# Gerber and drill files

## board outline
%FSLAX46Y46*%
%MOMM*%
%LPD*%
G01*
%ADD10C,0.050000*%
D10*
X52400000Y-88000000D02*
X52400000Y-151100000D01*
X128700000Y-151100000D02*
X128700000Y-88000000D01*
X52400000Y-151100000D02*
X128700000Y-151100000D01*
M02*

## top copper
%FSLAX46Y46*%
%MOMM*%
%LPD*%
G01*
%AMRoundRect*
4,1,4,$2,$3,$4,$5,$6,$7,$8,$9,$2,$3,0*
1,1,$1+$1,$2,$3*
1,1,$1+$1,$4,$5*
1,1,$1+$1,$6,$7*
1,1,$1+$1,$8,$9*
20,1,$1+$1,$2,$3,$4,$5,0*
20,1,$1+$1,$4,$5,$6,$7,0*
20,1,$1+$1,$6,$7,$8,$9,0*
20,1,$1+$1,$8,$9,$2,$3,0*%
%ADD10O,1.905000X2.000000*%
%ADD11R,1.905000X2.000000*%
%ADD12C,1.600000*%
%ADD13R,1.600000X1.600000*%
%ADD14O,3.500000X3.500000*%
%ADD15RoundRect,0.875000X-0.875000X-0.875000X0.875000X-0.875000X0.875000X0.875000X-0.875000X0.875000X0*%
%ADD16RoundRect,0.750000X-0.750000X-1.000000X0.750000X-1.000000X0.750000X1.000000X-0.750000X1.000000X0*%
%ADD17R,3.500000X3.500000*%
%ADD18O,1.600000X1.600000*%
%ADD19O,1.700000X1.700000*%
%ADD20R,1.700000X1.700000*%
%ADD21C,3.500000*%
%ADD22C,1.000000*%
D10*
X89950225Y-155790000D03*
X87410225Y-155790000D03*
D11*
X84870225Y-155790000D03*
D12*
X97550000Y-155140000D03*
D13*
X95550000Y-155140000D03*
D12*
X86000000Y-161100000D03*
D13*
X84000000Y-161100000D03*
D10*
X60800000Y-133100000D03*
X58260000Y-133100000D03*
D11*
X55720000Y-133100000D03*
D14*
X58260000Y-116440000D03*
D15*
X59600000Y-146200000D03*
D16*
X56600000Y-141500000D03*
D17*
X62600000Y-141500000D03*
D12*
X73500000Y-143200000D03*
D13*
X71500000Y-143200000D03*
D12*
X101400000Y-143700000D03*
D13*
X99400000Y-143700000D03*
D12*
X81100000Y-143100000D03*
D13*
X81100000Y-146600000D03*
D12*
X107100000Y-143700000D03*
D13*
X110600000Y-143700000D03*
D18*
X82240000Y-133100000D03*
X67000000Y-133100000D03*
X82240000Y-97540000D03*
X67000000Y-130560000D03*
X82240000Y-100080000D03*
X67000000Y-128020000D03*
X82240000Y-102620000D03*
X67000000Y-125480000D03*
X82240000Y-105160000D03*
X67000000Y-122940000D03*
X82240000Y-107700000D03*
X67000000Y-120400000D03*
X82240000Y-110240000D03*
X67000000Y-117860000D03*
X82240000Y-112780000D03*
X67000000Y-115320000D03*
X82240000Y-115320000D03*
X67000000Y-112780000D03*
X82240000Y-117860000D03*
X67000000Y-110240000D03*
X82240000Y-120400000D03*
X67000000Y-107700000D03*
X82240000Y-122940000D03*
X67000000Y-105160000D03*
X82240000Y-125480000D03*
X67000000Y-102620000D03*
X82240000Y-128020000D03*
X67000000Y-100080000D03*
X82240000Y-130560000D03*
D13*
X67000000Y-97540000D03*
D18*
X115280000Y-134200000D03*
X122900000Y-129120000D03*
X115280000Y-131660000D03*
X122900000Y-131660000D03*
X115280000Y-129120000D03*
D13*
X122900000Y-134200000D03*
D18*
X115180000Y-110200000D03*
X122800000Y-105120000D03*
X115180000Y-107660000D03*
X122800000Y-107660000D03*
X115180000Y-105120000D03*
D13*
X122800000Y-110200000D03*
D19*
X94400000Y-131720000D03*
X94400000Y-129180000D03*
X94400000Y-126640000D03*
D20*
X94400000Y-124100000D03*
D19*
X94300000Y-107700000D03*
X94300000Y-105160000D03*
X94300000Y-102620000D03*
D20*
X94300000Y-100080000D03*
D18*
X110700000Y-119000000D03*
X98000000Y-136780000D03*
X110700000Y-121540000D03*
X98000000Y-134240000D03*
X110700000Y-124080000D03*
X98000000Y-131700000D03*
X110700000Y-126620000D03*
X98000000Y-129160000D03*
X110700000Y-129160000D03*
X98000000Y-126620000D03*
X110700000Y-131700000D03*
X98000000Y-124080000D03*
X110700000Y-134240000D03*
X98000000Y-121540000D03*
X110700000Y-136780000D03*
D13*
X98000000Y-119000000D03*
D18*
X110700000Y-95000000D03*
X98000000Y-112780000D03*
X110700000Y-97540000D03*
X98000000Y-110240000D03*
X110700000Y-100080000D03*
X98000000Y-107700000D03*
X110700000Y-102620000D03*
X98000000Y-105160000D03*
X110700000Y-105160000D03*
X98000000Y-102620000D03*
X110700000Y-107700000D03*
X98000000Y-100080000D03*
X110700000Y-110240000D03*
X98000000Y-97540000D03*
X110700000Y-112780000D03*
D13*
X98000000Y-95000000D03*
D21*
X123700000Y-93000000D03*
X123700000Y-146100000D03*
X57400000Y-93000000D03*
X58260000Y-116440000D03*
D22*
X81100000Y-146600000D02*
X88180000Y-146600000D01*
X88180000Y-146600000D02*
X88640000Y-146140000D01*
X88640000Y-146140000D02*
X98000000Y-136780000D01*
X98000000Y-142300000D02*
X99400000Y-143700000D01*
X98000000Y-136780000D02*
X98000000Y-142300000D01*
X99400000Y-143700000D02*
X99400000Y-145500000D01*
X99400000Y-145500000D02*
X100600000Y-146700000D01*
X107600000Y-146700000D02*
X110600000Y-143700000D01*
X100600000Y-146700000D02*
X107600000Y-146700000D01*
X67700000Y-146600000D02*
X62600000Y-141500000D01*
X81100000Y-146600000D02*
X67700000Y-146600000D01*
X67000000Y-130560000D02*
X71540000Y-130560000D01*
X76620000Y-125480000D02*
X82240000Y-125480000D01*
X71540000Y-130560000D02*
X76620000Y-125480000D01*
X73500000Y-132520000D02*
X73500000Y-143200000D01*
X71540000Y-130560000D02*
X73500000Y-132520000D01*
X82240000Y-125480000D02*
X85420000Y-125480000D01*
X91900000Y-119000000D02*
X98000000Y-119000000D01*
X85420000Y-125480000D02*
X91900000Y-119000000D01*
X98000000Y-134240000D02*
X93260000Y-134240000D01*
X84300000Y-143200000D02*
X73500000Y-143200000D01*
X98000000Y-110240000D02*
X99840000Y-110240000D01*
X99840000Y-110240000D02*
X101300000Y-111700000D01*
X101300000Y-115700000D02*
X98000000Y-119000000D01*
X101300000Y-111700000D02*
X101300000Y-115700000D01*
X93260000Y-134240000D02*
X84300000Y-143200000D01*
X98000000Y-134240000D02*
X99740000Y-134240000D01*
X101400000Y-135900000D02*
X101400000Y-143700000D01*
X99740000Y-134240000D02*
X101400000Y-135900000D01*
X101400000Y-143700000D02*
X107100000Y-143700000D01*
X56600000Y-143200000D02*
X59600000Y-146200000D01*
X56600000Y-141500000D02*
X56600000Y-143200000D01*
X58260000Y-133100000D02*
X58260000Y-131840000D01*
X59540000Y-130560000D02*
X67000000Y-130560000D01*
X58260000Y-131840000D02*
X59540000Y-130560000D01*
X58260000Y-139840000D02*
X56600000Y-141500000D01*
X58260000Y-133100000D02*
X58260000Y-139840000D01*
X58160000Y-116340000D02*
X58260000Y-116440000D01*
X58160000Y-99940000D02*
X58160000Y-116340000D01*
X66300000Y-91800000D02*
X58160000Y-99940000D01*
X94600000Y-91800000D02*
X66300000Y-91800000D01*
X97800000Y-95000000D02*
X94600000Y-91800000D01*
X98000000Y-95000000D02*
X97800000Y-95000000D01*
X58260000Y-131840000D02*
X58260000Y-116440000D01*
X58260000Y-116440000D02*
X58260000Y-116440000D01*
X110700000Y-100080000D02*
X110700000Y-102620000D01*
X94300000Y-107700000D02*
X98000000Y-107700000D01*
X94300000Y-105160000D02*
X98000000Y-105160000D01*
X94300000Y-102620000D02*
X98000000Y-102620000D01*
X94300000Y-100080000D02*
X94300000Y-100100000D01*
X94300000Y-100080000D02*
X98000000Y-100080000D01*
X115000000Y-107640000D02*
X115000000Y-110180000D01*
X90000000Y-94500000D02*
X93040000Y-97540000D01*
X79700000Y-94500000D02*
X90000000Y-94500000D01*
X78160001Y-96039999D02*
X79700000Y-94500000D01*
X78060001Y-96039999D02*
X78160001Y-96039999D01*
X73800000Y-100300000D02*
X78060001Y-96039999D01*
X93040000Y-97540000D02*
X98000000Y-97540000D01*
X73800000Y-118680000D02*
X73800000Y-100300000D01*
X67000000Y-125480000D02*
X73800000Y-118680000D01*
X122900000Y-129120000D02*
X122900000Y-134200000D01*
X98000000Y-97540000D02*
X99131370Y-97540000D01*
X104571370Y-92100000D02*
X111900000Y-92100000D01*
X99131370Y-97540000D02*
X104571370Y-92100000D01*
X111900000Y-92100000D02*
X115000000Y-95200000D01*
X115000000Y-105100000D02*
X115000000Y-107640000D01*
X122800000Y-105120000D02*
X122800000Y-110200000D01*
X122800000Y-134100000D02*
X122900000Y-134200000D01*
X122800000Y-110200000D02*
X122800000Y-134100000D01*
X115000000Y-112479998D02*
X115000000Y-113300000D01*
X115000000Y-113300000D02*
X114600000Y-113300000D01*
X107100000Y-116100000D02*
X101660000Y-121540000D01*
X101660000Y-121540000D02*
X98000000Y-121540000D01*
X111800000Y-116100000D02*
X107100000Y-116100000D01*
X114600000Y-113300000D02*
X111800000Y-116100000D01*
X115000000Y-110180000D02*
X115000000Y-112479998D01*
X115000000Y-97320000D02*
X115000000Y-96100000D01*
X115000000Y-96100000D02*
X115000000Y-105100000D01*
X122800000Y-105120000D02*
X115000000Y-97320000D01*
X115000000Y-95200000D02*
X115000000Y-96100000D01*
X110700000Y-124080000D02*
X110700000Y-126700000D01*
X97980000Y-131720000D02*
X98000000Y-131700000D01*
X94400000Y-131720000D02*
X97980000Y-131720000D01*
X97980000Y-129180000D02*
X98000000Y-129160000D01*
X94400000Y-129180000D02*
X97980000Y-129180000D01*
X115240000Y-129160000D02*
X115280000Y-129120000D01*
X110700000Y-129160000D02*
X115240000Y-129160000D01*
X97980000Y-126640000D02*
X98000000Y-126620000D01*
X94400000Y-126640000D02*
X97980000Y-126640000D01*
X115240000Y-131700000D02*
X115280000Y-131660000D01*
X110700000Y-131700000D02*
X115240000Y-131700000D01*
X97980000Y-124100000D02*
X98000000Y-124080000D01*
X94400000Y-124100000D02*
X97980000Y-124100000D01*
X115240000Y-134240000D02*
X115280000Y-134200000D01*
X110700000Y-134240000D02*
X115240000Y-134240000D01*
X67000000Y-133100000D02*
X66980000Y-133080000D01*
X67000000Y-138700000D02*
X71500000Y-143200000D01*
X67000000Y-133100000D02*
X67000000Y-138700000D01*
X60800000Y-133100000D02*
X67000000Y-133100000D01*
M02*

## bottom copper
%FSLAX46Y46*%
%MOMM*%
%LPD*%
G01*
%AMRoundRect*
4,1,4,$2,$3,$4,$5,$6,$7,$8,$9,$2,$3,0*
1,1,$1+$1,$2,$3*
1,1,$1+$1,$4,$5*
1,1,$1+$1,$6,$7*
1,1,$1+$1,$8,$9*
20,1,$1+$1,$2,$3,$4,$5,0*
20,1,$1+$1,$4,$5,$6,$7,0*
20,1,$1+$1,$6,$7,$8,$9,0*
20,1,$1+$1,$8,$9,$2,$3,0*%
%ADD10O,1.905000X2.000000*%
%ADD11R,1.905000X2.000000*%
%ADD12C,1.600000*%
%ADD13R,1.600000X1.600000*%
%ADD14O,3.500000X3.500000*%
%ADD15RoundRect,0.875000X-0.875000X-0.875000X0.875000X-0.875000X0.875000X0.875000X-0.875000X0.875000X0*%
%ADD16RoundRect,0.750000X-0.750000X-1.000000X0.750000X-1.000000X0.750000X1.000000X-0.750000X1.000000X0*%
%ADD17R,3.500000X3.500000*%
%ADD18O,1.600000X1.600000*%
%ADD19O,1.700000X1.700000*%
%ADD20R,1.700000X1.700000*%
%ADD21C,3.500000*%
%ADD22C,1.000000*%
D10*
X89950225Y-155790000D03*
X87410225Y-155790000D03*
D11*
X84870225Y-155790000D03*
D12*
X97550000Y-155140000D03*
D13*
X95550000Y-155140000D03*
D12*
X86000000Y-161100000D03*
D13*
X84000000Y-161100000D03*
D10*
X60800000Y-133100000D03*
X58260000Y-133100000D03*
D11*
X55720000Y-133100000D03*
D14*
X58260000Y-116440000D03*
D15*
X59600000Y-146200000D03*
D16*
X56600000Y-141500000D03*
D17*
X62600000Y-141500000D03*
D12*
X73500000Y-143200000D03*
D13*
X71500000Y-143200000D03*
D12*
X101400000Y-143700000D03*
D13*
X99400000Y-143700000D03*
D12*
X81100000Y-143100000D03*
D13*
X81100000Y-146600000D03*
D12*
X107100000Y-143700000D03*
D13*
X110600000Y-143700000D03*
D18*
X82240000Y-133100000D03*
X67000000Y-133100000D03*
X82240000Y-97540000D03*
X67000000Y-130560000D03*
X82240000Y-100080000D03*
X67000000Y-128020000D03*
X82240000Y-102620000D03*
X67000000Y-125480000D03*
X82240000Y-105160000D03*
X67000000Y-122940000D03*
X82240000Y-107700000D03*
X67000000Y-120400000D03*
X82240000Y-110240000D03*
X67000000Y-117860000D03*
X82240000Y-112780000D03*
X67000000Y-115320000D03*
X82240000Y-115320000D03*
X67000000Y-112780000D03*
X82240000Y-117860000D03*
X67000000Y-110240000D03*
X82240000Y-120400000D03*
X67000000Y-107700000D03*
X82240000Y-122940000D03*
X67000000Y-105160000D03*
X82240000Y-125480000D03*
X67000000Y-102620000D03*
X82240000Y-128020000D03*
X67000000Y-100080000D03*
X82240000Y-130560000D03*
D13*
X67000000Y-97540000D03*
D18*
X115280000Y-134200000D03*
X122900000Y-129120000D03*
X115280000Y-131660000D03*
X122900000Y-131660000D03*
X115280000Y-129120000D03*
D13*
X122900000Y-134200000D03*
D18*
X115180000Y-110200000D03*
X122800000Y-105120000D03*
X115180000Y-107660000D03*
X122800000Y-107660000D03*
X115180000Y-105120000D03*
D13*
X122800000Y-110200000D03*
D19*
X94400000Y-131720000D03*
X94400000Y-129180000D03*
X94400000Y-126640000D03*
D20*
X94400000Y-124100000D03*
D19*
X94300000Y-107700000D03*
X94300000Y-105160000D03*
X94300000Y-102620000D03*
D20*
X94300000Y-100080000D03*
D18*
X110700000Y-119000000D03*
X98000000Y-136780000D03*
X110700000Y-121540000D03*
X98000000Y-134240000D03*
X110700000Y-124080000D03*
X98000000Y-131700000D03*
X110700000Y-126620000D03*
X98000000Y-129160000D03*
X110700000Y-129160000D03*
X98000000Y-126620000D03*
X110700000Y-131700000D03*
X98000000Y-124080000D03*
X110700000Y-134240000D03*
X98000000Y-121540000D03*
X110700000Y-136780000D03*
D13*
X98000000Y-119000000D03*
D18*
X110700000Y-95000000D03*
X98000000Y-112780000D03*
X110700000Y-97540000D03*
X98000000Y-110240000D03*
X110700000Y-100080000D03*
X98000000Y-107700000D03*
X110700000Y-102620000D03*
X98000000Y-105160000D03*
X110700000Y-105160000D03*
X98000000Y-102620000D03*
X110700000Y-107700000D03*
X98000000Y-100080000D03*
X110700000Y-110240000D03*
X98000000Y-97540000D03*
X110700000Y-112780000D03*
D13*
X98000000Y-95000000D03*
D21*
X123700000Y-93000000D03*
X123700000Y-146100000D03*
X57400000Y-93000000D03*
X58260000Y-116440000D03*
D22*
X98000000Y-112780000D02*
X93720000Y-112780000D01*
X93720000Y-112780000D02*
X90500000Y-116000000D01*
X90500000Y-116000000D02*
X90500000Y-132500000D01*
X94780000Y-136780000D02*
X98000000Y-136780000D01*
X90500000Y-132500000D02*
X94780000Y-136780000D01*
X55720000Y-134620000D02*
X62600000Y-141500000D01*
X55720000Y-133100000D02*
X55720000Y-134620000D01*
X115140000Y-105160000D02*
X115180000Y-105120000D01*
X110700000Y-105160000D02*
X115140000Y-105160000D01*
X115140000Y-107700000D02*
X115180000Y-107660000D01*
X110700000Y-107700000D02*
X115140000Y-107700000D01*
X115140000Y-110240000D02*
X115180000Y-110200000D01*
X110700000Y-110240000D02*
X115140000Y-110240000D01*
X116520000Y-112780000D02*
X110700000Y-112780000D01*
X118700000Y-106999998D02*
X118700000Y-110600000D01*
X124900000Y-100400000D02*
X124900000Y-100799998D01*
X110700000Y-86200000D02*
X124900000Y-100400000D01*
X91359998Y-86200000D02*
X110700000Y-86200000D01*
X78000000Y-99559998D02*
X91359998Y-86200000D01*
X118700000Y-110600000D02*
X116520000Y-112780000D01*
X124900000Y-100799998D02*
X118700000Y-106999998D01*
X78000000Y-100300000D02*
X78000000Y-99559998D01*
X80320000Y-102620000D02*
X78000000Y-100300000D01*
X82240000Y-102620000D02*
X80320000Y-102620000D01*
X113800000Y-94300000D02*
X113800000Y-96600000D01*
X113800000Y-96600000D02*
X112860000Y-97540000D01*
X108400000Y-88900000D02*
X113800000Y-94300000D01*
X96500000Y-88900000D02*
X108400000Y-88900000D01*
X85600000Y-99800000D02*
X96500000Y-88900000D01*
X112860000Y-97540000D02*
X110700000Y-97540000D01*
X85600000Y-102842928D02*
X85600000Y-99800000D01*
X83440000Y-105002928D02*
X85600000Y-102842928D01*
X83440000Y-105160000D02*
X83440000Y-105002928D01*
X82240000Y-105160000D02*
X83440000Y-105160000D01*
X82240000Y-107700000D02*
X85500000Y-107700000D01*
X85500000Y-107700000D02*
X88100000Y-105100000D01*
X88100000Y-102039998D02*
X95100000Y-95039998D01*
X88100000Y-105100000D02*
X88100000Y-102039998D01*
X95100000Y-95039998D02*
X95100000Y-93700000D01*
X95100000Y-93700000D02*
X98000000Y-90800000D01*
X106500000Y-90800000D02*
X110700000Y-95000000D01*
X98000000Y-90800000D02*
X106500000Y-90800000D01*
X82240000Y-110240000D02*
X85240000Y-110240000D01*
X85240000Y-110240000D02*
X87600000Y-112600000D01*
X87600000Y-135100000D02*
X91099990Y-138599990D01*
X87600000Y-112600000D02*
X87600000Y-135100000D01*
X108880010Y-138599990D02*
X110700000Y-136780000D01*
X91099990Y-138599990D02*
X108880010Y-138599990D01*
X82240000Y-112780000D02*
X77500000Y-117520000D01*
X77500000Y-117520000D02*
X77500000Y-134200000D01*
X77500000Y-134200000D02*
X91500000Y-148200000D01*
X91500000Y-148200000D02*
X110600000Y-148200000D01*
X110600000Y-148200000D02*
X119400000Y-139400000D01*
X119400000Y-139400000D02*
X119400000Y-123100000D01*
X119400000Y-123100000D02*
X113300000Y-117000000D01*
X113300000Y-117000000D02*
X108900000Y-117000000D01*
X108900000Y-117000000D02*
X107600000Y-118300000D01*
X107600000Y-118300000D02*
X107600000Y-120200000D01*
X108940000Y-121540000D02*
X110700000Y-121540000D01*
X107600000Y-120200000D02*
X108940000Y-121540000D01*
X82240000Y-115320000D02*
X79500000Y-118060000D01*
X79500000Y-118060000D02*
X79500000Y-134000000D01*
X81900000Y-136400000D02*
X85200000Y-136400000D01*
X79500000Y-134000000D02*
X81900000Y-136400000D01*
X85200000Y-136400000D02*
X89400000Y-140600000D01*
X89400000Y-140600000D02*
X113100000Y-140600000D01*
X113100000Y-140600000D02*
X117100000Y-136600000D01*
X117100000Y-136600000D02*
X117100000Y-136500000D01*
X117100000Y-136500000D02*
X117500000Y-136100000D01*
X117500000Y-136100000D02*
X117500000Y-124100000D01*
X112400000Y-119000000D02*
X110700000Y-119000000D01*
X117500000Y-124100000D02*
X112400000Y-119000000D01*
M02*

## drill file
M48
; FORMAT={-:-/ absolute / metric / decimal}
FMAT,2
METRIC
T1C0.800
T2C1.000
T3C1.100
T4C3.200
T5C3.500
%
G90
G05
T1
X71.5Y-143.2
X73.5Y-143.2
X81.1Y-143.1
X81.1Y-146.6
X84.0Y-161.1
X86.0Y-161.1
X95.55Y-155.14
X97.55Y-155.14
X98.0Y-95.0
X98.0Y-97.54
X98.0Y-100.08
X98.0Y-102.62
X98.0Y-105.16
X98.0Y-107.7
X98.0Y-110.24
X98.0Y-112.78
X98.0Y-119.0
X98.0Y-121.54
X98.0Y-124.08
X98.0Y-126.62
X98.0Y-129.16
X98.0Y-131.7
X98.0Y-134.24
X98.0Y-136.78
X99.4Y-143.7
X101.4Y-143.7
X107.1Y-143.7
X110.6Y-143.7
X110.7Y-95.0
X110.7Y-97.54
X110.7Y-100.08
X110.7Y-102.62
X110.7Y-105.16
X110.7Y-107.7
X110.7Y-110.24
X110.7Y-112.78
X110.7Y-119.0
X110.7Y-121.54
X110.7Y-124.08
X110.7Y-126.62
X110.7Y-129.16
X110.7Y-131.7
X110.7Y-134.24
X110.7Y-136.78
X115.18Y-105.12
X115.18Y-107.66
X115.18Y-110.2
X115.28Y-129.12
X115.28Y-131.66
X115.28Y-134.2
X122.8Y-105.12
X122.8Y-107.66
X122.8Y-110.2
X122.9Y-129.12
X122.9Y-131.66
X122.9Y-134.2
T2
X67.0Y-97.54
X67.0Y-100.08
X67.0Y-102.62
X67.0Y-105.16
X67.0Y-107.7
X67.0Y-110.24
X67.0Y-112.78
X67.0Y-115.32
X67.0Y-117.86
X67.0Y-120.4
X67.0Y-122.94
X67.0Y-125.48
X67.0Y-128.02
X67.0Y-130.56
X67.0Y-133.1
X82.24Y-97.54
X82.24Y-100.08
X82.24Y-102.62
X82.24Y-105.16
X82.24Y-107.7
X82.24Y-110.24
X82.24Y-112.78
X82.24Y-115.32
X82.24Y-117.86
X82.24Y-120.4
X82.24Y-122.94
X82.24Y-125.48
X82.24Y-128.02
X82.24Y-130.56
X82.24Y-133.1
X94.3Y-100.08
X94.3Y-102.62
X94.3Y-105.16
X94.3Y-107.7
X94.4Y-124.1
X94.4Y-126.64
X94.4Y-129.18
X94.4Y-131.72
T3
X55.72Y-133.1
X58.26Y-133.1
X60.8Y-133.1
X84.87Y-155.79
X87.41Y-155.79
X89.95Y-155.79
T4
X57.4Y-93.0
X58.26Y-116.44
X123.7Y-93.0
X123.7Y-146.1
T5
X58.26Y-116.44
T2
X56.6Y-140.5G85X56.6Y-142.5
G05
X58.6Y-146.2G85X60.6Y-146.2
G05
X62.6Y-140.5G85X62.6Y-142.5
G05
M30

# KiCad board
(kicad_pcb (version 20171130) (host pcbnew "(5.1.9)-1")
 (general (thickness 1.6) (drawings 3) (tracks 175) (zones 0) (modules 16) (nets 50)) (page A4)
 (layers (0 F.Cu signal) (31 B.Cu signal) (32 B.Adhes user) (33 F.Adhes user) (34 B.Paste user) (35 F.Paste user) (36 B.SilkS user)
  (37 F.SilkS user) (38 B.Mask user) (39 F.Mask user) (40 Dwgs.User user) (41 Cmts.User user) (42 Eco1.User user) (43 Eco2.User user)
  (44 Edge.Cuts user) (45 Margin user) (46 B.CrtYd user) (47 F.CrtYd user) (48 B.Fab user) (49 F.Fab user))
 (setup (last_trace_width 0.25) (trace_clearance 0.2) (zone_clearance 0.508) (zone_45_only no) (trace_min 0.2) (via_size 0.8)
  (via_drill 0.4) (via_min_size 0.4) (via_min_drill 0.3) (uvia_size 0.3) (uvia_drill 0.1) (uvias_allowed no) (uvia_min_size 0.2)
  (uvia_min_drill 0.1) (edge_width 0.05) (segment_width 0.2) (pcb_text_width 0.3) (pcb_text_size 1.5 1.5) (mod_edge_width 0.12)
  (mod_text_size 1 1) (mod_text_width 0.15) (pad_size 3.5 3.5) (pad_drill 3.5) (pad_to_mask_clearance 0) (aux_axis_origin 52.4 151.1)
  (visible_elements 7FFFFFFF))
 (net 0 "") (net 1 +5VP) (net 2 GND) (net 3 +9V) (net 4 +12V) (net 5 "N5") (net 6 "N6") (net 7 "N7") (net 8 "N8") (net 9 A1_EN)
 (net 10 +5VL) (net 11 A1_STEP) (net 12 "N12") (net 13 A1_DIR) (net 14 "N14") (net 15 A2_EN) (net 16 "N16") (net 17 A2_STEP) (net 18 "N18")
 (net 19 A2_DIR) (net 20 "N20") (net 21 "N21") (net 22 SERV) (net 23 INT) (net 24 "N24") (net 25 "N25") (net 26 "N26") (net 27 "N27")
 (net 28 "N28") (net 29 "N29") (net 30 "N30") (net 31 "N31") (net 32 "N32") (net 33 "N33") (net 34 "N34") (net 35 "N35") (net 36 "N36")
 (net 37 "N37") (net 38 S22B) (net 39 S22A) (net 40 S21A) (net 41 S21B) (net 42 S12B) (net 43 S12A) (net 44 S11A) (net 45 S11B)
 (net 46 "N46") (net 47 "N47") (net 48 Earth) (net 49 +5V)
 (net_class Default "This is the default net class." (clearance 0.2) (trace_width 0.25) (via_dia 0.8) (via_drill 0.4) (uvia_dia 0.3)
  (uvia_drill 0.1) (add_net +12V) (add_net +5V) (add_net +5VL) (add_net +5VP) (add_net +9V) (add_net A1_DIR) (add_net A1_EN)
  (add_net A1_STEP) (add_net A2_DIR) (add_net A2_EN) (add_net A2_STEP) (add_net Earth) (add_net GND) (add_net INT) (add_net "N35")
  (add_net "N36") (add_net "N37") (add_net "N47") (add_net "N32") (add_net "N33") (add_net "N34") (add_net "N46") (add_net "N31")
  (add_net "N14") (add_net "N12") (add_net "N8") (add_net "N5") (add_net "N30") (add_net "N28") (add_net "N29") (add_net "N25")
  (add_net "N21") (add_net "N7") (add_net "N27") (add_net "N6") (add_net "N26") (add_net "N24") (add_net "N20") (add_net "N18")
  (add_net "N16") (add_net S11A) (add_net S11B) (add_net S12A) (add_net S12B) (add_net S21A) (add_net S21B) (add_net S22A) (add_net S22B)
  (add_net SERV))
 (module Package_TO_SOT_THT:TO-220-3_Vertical (layer F.Cu) (at 84.870225 155.79)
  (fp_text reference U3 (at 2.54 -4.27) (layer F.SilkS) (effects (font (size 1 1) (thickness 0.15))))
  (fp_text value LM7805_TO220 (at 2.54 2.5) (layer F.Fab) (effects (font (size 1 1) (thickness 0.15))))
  (pad 3 thru_hole oval (at 5.08 0) (size 1.905 2) (drill 1.1) (layers *.Cu *.Mask) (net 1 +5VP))
  (pad 2 thru_hole oval (at 2.54 0) (size 1.905 2) (drill 1.1) (layers *.Cu *.Mask) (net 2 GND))
  (pad 1 thru_hole rect (at 0 0) (size 1.905 2) (drill 1.1) (layers *.Cu *.Mask) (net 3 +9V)))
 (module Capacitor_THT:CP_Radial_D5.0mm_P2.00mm (layer F.Cu) (at 95.55 155.14)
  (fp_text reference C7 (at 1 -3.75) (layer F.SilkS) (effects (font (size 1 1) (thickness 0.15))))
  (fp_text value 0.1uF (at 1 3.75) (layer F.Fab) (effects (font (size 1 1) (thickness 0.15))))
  (pad 2 thru_hole circle (at 2 0) (size 1.6 1.6) (drill 0.8) (layers *.Cu *.Mask) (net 2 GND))
  (pad 1 thru_hole rect (at 0 0) (size 1.6 1.6) (drill 0.8) (layers *.Cu *.Mask) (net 1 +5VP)))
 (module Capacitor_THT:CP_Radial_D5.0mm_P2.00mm (layer F.Cu) (at 84 161.1)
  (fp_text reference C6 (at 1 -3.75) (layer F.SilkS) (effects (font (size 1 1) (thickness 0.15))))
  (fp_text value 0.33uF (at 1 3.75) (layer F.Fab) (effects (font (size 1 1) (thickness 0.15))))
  (pad 2 thru_hole circle (at 2 0) (size 1.6 1.6) (drill 0.8) (layers *.Cu *.Mask) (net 2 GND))
  (pad 1 thru_hole rect (at 0 0) (size 1.6 1.6) (drill 0.8) (layers *.Cu *.Mask) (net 3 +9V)))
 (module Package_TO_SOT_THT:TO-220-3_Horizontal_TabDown (layer F.Cu) (at 55.72 133.1)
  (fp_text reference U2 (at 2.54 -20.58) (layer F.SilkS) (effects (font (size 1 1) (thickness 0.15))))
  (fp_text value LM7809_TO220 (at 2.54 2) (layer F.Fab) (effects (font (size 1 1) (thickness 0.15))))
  (pad 3 thru_hole oval (at 5.08 0) (size 1.905 2) (drill 1.1) (layers *.Cu *.Mask) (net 3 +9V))
  (pad 2 thru_hole oval (at 2.54 0) (size 1.905 2) (drill 1.1) (layers *.Cu *.Mask) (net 2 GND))
  (pad 1 thru_hole rect (at 0 0) (size 1.905 2) (drill 1.1) (layers *.Cu *.Mask) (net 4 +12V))
  (pad "" thru_hole oval (at 2.54 -16.66) (size 3.5 3.5) (drill 3.5) (layers *.Cu *.Mask)))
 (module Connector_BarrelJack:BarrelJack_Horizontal (layer F.Cu) (at 62.6 141.5)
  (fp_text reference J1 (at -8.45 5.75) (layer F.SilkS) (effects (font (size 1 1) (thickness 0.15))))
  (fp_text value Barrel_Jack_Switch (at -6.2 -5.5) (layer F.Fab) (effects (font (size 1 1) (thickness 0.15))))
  (pad 3 thru_hole roundrect (at -3 4.7) (size 3.5 3.5) (drill oval 3 1) (layers *.Cu *.Mask) (roundrect_rratio 0.25) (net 2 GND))
  (pad 2 thru_hole roundrect (at -6 0) (size 3 3.5) (drill oval 1 3) (layers *.Cu *.Mask) (roundrect_rratio 0.25) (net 2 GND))
  (pad 1 thru_hole rect (at 0 0) (size 3.5 3.5) (drill oval 1 3) (layers *.Cu *.Mask) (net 4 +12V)))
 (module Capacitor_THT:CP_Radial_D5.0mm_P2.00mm (layer F.Cu) (at 71.5 143.2)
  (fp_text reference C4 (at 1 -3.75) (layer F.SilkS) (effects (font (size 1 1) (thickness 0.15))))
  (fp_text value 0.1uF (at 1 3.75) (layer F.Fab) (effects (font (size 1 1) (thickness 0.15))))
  (pad 2 thru_hole circle (at 2 0) (size 1.6 1.6) (drill 0.8) (layers *.Cu *.Mask) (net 2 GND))
  (pad 1 thru_hole rect (at 0 0) (size 1.6 1.6) (drill 0.8) (layers *.Cu *.Mask) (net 3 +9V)))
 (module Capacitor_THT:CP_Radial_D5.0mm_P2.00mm (layer F.Cu) (at 99.4 143.7)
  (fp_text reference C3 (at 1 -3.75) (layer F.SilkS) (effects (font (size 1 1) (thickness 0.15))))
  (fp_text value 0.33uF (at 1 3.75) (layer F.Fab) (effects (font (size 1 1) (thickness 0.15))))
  (pad 2 thru_hole circle (at 2 0) (size 1.6 1.6) (drill 0.8) (layers *.Cu *.Mask) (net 2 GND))
  (pad 1 thru_hole rect (at 0 0) (size 1.6 1.6) (drill 0.8) (layers *.Cu *.Mask) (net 4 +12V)))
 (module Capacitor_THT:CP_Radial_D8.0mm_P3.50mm (layer F.Cu) (at 81.1 146.6 90)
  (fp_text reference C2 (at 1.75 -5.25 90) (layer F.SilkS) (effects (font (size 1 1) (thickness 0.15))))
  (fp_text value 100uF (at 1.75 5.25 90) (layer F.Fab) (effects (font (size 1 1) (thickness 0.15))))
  (pad 2 thru_hole circle (at 3.5 0 90) (size 1.6 1.6) (drill 0.8) (layers *.Cu *.Mask) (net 2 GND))
  (pad 1 thru_hole rect (at 0 0 90) (size 1.6 1.6) (drill 0.8) (layers *.Cu *.Mask) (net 4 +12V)))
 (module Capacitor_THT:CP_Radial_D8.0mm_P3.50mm (layer F.Cu) (at 110.6 143.7 180)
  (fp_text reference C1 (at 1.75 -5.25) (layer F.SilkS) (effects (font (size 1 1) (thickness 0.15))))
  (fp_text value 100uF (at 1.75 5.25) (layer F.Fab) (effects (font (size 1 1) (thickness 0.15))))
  (pad 2 thru_hole circle (at 3.5 0 180) (size 1.6 1.6) (drill 0.8) (layers *.Cu *.Mask) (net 2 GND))
  (pad 1 thru_hole rect (at 0 0 180) (size 1.6 1.6) (drill 0.8) (layers *.Cu *.Mask) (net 4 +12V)))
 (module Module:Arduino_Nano (layer F.Cu) (at 67 97.54)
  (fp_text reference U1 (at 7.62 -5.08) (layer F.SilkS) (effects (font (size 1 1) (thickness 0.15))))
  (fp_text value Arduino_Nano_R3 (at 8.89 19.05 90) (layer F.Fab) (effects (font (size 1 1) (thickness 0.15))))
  (pad 16 thru_hole oval (at 15.24 35.56) (size 1.6 1.6) (drill 1) (layers *.Cu *.Mask) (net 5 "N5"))
  (pad 15 thru_hole oval (at 0 35.56) (size 1.6 1.6) (drill 1) (layers *.Cu *.Mask) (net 3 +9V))
  (pad 30 thru_hole oval (at 15.24 0) (size 1.6 1.6) (drill 1) (layers *.Cu *.Mask) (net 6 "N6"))
  (pad 14 thru_hole oval (at 0 33.02) (size 1.6 1.6) (drill 1) (layers *.Cu *.Mask) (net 2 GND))
  (pad 29 thru_hole oval (at 15.24 2.54) (size 1.6 1.6) (drill 1) (layers *.Cu *.Mask) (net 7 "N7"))
  (pad 13 thru_hole oval (at 0 30.48) (size 1.6 1.6) (drill 1) (layers *.Cu *.Mask) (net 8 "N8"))
  (pad 28 thru_hole oval (at 15.24 5.08) (size 1.6 1.6) (drill 1) (layers *.Cu *.Mask) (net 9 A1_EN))
  (pad 12 thru_hole oval (at 0 27.94) (size 1.6 1.6) (drill 1) (layers *.Cu *.Mask) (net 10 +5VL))
  (pad 27 thru_hole oval (at 15.24 7.62) (size 1.6 1.6) (drill 1) (layers *.Cu *.Mask) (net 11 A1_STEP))
  (pad 11 thru_hole oval (at 0 25.4) (size 1.6 1.6) (drill 1) (layers *.Cu *.Mask) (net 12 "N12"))
  (pad 26 thru_hole oval (at 15.24 10.16) (size 1.6 1.6) (drill 1) (layers *.Cu *.Mask) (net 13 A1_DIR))
  (pad 10 thru_hole oval (at 0 22.86) (size 1.6 1.6) (drill 1) (layers *.Cu *.Mask) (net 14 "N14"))
  (pad 25 thru_hole oval (at 15.24 12.7) (size 1.6 1.6) (drill 1) (layers *.Cu *.Mask) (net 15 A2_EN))
  (pad 9 thru_hole oval (at 0 20.32) (size 1.6 1.6) (drill 1) (layers *.Cu *.Mask) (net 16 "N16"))
  (pad 24 thru_hole oval (at 15.24 15.24) (size 1.6 1.6) (drill 1) (layers *.Cu *.Mask) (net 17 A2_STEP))
  (pad 8 thru_hole oval (at 0 17.78) (size 1.6 1.6) (drill 1) (layers *.Cu *.Mask) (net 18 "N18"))
  (pad 23 thru_hole oval (at 15.24 17.78) (size 1.6 1.6) (drill 1) (layers *.Cu *.Mask) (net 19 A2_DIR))
  (pad 7 thru_hole oval (at 0 15.24) (size 1.6 1.6) (drill 1) (layers *.Cu *.Mask) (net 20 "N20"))
  (pad 22 thru_hole oval (at 15.24 20.32) (size 1.6 1.6) (drill 1) (layers *.Cu *.Mask) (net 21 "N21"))
  (pad 6 thru_hole oval (at 0 12.7) (size 1.6 1.6) (drill 1) (layers *.Cu *.Mask) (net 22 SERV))
  (pad 21 thru_hole oval (at 15.24 22.86) (size 1.6 1.6) (drill 1) (layers *.Cu *.Mask) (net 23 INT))
  (pad 5 thru_hole oval (at 0 10.16) (size 1.6 1.6) (drill 1) (layers *.Cu *.Mask) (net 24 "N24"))
  (pad 20 thru_hole oval (at 15.24 25.4) (size 1.6 1.6) (drill 1) (layers *.Cu *.Mask) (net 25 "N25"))
  (pad 4 thru_hole oval (at 0 7.62) (size 1.6 1.6) (drill 1) (layers *.Cu *.Mask) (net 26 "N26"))
  (pad 19 thru_hole oval (at 15.24 27.94) (size 1.6 1.6) (drill 1) (layers *.Cu *.Mask) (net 2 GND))
  (pad 3 thru_hole oval (at 0 5.08) (size 1.6 1.6) (drill 1) (layers *.Cu *.Mask) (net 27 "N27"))
  (pad 18 thru_hole oval (at 15.24 30.48) (size 1.6 1.6) (drill 1) (layers *.Cu *.Mask) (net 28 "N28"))
  (pad 2 thru_hole oval (at 0 2.54) (size 1.6 1.6) (drill 1) (layers *.Cu *.Mask) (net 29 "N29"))
  (pad 17 thru_hole oval (at 15.24 33.02) (size 1.6 1.6) (drill 1) (layers *.Cu *.Mask) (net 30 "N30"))
  (pad 1 thru_hole rect (at 0 0) (size 1.6 1.6) (drill 1) (layers *.Cu *.Mask) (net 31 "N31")))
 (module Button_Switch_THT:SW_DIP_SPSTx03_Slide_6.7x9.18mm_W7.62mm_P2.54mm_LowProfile (layer F.Cu) (at 122.9 134.2 180)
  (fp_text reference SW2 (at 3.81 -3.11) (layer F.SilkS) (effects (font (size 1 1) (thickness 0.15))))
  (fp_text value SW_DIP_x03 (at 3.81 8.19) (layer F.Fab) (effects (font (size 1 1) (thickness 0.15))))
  (pad 6 thru_hole oval (at 7.62 0 180) (size 1.6 1.6) (drill 0.8) (layers *.Cu *.Mask) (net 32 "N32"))
  (pad 3 thru_hole oval (at 0 5.08 180) (size 1.6 1.6) (drill 0.8) (layers *.Cu *.Mask) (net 10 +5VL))
  (pad 5 thru_hole oval (at 7.62 2.54 180) (size 1.6 1.6) (drill 0.8) (layers *.Cu *.Mask) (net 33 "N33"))
  (pad 2 thru_hole oval (at 0 2.54 180) (size 1.6 1.6) (drill 0.8) (layers *.Cu *.Mask) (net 10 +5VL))
  (pad 4 thru_hole oval (at 7.62 5.08 180) (size 1.6 1.6) (drill 0.8) (layers *.Cu *.Mask) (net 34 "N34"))
  (pad 1 thru_hole rect (at 0 0 180) (size 1.6 1.6) (drill 0.8) (layers *.Cu *.Mask) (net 10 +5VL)))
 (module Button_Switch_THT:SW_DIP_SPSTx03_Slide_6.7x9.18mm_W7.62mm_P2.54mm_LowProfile (layer F.Cu) (at 122.8 110.2 180)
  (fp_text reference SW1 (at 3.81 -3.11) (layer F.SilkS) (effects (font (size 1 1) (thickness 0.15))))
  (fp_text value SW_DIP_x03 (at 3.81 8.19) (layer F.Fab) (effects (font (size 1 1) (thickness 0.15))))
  (pad 6 thru_hole oval (at 7.62 0 180) (size 1.6 1.6) (drill 0.8) (layers *.Cu *.Mask) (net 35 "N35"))
  (pad 3 thru_hole oval (at 0 5.08 180) (size 1.6 1.6) (drill 0.8) (layers *.Cu *.Mask) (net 10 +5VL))
  (pad 5 thru_hole oval (at 7.62 2.54 180) (size 1.6 1.6) (drill 0.8) (layers *.Cu *.Mask) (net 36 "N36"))
  (pad 2 thru_hole oval (at 0 2.54 180) (size 1.6 1.6) (drill 0.8) (layers *.Cu *.Mask) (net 10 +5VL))
  (pad 4 thru_hole oval (at 7.62 5.08 180) (size 1.6 1.6) (drill 0.8) (layers *.Cu *.Mask) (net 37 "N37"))
  (pad 1 thru_hole rect (at 0 0 180) (size 1.6 1.6) (drill 0.8) (layers *.Cu *.Mask) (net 10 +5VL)))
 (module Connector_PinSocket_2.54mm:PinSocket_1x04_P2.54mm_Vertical (layer F.Cu) (at 94.4 124.1)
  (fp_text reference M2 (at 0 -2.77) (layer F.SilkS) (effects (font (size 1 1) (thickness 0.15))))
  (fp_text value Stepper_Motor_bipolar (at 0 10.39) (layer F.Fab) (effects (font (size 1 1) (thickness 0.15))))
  (pad 4 thru_hole oval (at 0 7.62) (size 1.7 1.7) (drill 1) (layers *.Cu *.Mask) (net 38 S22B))
  (pad 3 thru_hole oval (at 0 5.08) (size 1.7 1.7) (drill 1) (layers *.Cu *.Mask) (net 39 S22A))
  (pad 2 thru_hole oval (at 0 2.54) (size 1.7 1.7) (drill 1) (layers *.Cu *.Mask) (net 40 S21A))
  (pad 1 thru_hole rect (at 0 0) (size 1.7 1.7) (drill 1) (layers *.Cu *.Mask) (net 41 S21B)))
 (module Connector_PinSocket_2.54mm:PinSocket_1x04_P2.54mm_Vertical (layer F.Cu) (at 94.3 100.08)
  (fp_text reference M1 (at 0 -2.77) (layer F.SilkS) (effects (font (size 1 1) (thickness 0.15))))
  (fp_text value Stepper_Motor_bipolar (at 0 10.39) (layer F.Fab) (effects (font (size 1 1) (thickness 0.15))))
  (pad 4 thru_hole oval (at 0 7.62) (size 1.7 1.7) (drill 1) (layers *.Cu *.Mask) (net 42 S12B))
  (pad 3 thru_hole oval (at 0 5.08) (size 1.7 1.7) (drill 1) (layers *.Cu *.Mask) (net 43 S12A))
  (pad 2 thru_hole oval (at 0 2.54) (size 1.7 1.7) (drill 1) (layers *.Cu *.Mask) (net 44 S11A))
  (pad 1 thru_hole rect (at 0 0) (size 1.7 1.7) (drill 1) (layers *.Cu *.Mask) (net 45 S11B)))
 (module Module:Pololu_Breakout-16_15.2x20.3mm (layer F.Cu) (at 98 119)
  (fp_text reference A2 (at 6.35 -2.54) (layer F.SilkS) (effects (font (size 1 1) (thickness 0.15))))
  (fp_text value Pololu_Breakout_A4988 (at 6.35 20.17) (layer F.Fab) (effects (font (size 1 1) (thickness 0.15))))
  (pad 16 thru_hole oval (at 12.7 0) (size 1.6 1.6) (drill 0.8) (layers *.Cu *.Mask) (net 19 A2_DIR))
  (pad 8 thru_hole oval (at 0 17.78) (size 1.6 1.6) (drill 0.8) (layers *.Cu *.Mask) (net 4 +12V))
  (pad 15 thru_hole oval (at 12.7 2.54) (size 1.6 1.6) (drill 0.8) (layers *.Cu *.Mask) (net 17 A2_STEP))
  (pad 7 thru_hole oval (at 0 15.24) (size 1.6 1.6) (drill 0.8) (layers *.Cu *.Mask) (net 2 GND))
  (pad 14 thru_hole oval (at 12.7 5.08) (size 1.6 1.6) (drill 0.8) (layers *.Cu *.Mask) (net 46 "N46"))
  (pad 6 thru_hole oval (at 0 12.7) (size 1.6 1.6) (drill 0.8) (layers *.Cu *.Mask) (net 38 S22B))
  (pad 13 thru_hole oval (at 12.7 7.62) (size 1.6 1.6) (drill 0.8) (layers *.Cu *.Mask) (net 46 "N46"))
  (pad 5 thru_hole oval (at 0 10.16) (size 1.6 1.6) (drill 0.8) (layers *.Cu *.Mask) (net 39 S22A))
  (pad 12 thru_hole oval (at 12.7 10.16) (size 1.6 1.6) (drill 0.8) (layers *.Cu *.Mask) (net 34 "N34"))
  (pad 4 thru_hole oval (at 0 7.62) (size 1.6 1.6) (drill 0.8) (layers *.Cu *.Mask) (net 40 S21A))
  (pad 11 thru_hole oval (at 12.7 12.7) (size 1.6 1.6) (drill 0.8) (layers *.Cu *.Mask) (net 33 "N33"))
  (pad 3 thru_hole oval (at 0 5.08) (size 1.6 1.6) (drill 0.8) (layers *.Cu *.Mask) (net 41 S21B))
  (pad 10 thru_hole oval (at 12.7 15.24) (size 1.6 1.6) (drill 0.8) (layers *.Cu *.Mask) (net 32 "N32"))
  (pad 2 thru_hole oval (at 0 2.54) (size 1.6 1.6) (drill 0.8) (layers *.Cu *.Mask) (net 10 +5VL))
  (pad 9 thru_hole oval (at 12.7 17.78) (size 1.6 1.6) (drill 0.8) (layers *.Cu *.Mask) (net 15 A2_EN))
  (pad 1 thru_hole rect (at 0 0) (size 1.6 1.6) (drill 0.8) (layers *.Cu *.Mask) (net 2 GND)))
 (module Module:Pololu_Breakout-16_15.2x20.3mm (layer F.Cu) (at 98 95)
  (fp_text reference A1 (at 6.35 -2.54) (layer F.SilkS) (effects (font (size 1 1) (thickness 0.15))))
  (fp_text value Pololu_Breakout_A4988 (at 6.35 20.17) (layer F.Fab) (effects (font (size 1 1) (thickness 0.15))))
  (pad 16 thru_hole oval (at 12.7 0) (size 1.6 1.6) (drill 0.8) (layers *.Cu *.Mask) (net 13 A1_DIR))
  (pad 8 thru_hole oval (at 0 17.78) (size 1.6 1.6) (drill 0.8) (layers *.Cu *.Mask) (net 4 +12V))
  (pad 15 thru_hole oval (at 12.7 2.54) (size 1.6 1.6) (drill 0.8) (layers *.Cu *.Mask) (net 11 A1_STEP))
  (pad 7 thru_hole oval (at 0 15.24) (size 1.6 1.6) (drill 0.8) (layers *.Cu *.Mask) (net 2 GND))
  (pad 14 thru_hole oval (at 12.7 5.08) (size 1.6 1.6) (drill 0.8) (layers *.Cu *.Mask) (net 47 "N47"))
  (pad 6 thru_hole oval (at 0 12.7) (size 1.6 1.6) (drill 0.8) (layers *.Cu *.Mask) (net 42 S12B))
  (pad 13 thru_hole oval (at 12.7 7.62) (size 1.6 1.6) (drill 0.8) (layers *.Cu *.Mask) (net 47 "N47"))
  (pad 5 thru_hole oval (at 0 10.16) (size 1.6 1.6) (drill 0.8) (layers *.Cu *.Mask) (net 43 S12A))
  (pad 12 thru_hole oval (at 12.7 10.16) (size 1.6 1.6) (drill 0.8) (layers *.Cu *.Mask) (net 37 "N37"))
  (pad 4 thru_hole oval (at 0 7.62) (size 1.6 1.6) (drill 0.8) (layers *.Cu *.Mask) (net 44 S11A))
  (pad 11 thru_hole oval (at 12.7 12.7) (size 1.6 1.6) (drill 0.8) (layers *.Cu *.Mask) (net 36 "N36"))
  (pad 3 thru_hole oval (at 0 5.08) (size 1.6 1.6) (drill 0.8) (layers *.Cu *.Mask) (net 45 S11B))
  (pad 10 thru_hole oval (at 12.7 15.24) (size 1.6 1.6) (drill 0.8) (layers *.Cu *.Mask) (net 35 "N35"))
  (pad 2 thru_hole oval (at 0 2.54) (size 1.6 1.6) (drill 0.8) (layers *.Cu *.Mask) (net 10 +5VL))
  (pad 9 thru_hole oval (at 12.7 17.78) (size 1.6 1.6) (drill 0.8) (layers *.Cu *.Mask) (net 9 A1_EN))
  (pad 1 thru_hole rect (at 0 0) (size 1.6 1.6) (drill 0.8) (layers *.Cu *.Mask) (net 2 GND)))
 (gr_line (start 52.4 88) (end 52.4 151.1) (layer Edge.Cuts) (width 0.05))
 (gr_line (start 128.7 151.1) (end 128.7 88) (layer Edge.Cuts) (width 0.05))
 (gr_line (start 52.4 151.1) (end 128.7 151.1) (layer Edge.Cuts) (width 0.05))
 (segment (start 98 112.78) (end 93.72 112.78) (width 1) (layer B.Cu) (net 4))
 (segment (start 93.72 112.78) (end 90.5 116) (width 1) (layer B.Cu) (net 4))
 (segment (start 90.5 116) (end 90.5 132.5) (width 1) (layer B.Cu) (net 4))
 (segment (start 94.78 136.78) (end 98 136.78) (width 1) (layer B.Cu) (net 4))
 (segment (start 90.5 132.5) (end 94.78 136.78) (width 1) (layer B.Cu) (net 4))
 (segment (start 81.1 146.6) (end 88.18 146.6) (width 1) (layer F.Cu) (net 4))
 (segment (start 88.18 146.6) (end 88.64 146.14) (width 1) (layer F.Cu) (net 4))
 (segment (start 88.64 146.14) (end 98 136.78) (width 1) (layer F.Cu) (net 4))
 (segment (start 98 142.3) (end 99.4 143.7) (width 1) (layer F.Cu) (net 4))
 (segment (start 98 136.78) (end 98 142.3) (width 1) (layer F.Cu) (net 4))
 (segment (start 99.4 143.7) (end 99.4 145.5) (width 1) (layer F.Cu) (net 4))
 (segment (start 99.4 145.5) (end 100.6 146.7) (width 1) (layer F.Cu) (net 4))
 (segment (start 107.6 146.7) (end 110.6 143.7) (width 1) (layer F.Cu) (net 4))
 (segment (start 100.6 146.7) (end 107.6 146.7) (width 1) (layer F.Cu) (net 4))
 (segment (start 55.72 134.62) (end 62.6 141.5) (width 1) (layer B.Cu) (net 4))
 (segment (start 55.72 133.1) (end 55.72 134.62) (width 1) (layer B.Cu) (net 4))
 (segment (start 67.7 146.6) (end 62.6 141.5) (width 1) (layer F.Cu) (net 4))
 (segment (start 81.1 146.6) (end 67.7 146.6) (width 1) (layer F.Cu) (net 4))
 (via (at 123.7 93) (size 3.5) (drill 3.2) (layers F.Cu B.Cu) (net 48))
 (via (at 123.7 146.1) (size 3.5) (drill 3.2) (layers F.Cu B.Cu) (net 48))
 (via (at 57.4 93) (size 3.5) (drill 3.2) (layers F.Cu B.Cu) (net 48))
 (segment (start 67 130.56) (end 71.54 130.56) (width 1) (layer F.Cu) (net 48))
 (segment (start 76.62 125.48) (end 82.24 125.48) (width 1) (layer F.Cu) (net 48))
 (segment (start 71.54 130.56) (end 76.62 125.48) (width 1) (layer F.Cu) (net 48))
 (segment (start 73.5 132.52) (end 73.5 143.2) (width 1) (layer F.Cu) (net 48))
 (segment (start 71.54 130.56) (end 73.5 132.52) (width 1) (layer F.Cu) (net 48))
 (segment (start 82.24 125.48) (end 85.42 125.48) (width 1) (layer F.Cu) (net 48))
 (segment (start 91.9 119) (end 98 119) (width 1) (layer F.Cu) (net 48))
 (segment (start 85.42 125.48) (end 91.9 119) (width 1) (layer F.Cu) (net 48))
 (segment (start 98 134.24) (end 93.26 134.24) (width 1) (layer F.Cu) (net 48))
 (segment (start 84.3 143.2) (end 73.5 143.2) (width 1) (layer F.Cu) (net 48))
 (segment (start 98 110.24) (end 99.84 110.24) (width 1) (layer F.Cu) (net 48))
 (segment (start 99.84 110.24) (end 101.3 111.7) (width 1) (layer F.Cu) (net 48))
 (segment (start 101.3 115.7) (end 98 119) (width 1) (layer F.Cu) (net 48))
 (segment (start 101.3 111.7) (end 101.3 115.7) (width 1) (layer F.Cu) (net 48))
 (segment (start 93.26 134.24) (end 84.3 143.2) (width 1) (layer F.Cu) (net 48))
 (segment (start 98 134.24) (end 99.74 134.24) (width 1) (layer F.Cu) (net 48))
 (segment (start 101.4 135.9) (end 101.4 143.7) (width 1) (layer F.Cu) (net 48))
 (segment (start 99.74 134.24) (end 101.4 135.9) (width 1) (layer F.Cu) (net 48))
 (segment (start 101.4 143.7) (end 107.1 143.7) (width 1) (layer F.Cu) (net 48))
 (segment (start 56.6 143.2) (end 59.6 146.2) (width 1) (layer F.Cu) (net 48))
 (segment (start 56.6 141.5) (end 56.6 143.2) (width 1) (layer F.Cu) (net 48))
 (segment (start 58.26 133.1) (end 58.26 131.84) (width 1) (layer F.Cu) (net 48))
 (segment (start 59.54 130.56) (end 67 130.56) (width 1) (layer F.Cu) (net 48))
 (segment (start 58.26 131.84) (end 59.54 130.56) (width 1) (layer F.Cu) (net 48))
 (segment (start 58.26 139.84) (end 56.6 141.5) (width 1) (layer F.Cu) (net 48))
 (segment (start 58.26 133.1) (end 58.26 139.84) (width 1) (layer F.Cu) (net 48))
 (segment (start 58.16 116.34) (end 58.26 116.44) (width 1) (layer F.Cu) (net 48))
 (segment (start 58.16 99.94) (end 58.16 116.34) (width 1) (layer F.Cu) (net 48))
 (segment (start 66.3 91.8) (end 58.16 99.94) (width 1) (layer F.Cu) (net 48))
 (segment (start 94.6 91.8) (end 66.3 91.8) (width 1) (layer F.Cu) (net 48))
 (segment (start 97.8 95) (end 94.6 91.8) (width 1) (layer F.Cu) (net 48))
 (segment (start 98 95) (end 97.8 95) (width 1) (layer F.Cu) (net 48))
 (segment (start 58.26 131.84) (end 58.26 116.44) (width 1) (layer F.Cu) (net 48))
 (segment (start 58.26 116.44) (end 58.26 116.44) (width 1) (layer F.Cu) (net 48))
 (via (at 58.26 116.44) (size 3.5) (drill 3.2) (layers F.Cu B.Cu) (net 48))
 (segment (start 110.7 100.08) (end 110.7 102.62) (width 1) (layer F.Cu) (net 47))
 (segment (start 94.3 107.7) (end 98 107.7) (width 1) (layer F.Cu) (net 42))
 (segment (start 94.3 105.16) (end 98 105.16) (width 1) (layer F.Cu) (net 43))
 (segment (start 115.14 105.16) (end 115.18 105.12) (width 1) (layer B.Cu) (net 37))
 (segment (start 110.7 105.16) (end 115.14 105.16) (width 1) (layer B.Cu) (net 37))
 (segment (start 94.3 102.62) (end 98 102.62) (width 1) (layer F.Cu) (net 44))
 (segment (start 115.14 107.7) (end 115.18 107.66) (width 1) (layer B.Cu) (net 36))
 (segment (start 110.7 107.7) (end 115.14 107.7) (width 1) (layer B.Cu) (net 36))
 (segment (start 94.3 100.08) (end 94.3 100.1) (width 1) (layer F.Cu) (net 45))
 (segment (start 94.3 100.08) (end 98 100.08) (width 1) (layer F.Cu) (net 45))
 (segment (start 115.14 110.24) (end 115.18 110.2) (width 1) (layer B.Cu) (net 35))
 (segment (start 110.7 110.24) (end 115.14 110.24) (width 1) (layer B.Cu) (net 35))
 (segment (start 115 107.64) (end 115 110.18) (width 1) (layer F.Cu) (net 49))
 (segment (start 90 94.5) (end 93.04 97.54) (width 1) (layer F.Cu) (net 49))
 (segment (start 79.7 94.5) (end 90 94.5) (width 1) (layer F.Cu) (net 49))
 (segment (start 78.160001 96.039999) (end 79.7 94.5) (width 1) (layer F.Cu) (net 49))
 (segment (start 78.060001 96.039999) (end 78.160001 96.039999) (width 1) (layer F.Cu) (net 49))
 (segment (start 73.8 100.3) (end 78.060001 96.039999) (width 1) (layer F.Cu) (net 49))
 (segment (start 93.04 97.54) (end 98 97.54) (width 1) (layer F.Cu) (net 49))
 (segment (start 73.8 118.68) (end 73.8 100.3) (width 1) (layer F.Cu) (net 49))
 (segment (start 67 125.48) (end 73.8 118.68) (width 1) (layer F.Cu) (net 49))
 (segment (start 122.9 129.12) (end 122.9 134.2) (width 1) (layer F.Cu) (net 49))
 (segment (start 98 97.54) (end 99.13137 97.54) (width 1) (layer F.Cu) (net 49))
 (segment (start 104.57137 92.1) (end 111.9 92.1) (width 1) (layer F.Cu) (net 49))
 (segment (start 99.13137 97.54) (end 104.57137 92.1) (width 1) (layer F.Cu) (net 49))
 (segment (start 111.9 92.1) (end 115 95.2) (width 1) (layer F.Cu) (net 49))
 (segment (start 115 105.1) (end 115 107.64) (width 1) (layer F.Cu) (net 49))
 (segment (start 122.8 105.12) (end 122.8 110.2) (width 1) (layer F.Cu) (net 49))
 (segment (start 122.8 134.1) (end 122.9 134.2) (width 1) (layer F.Cu) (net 49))
 (segment (start 122.8 110.2) (end 122.8 134.1) (width 1) (layer F.Cu) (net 49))
 (segment (start 115 112.479998) (end 115 113.3) (width 1) (layer F.Cu) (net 49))
 (segment (start 115 113.3) (end 114.6 113.3) (width 1) (layer F.Cu) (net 49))
 (segment (start 107.1 116.1) (end 101.66 121.54) (width 1) (layer F.Cu) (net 49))
 (segment (start 101.66 121.54) (end 98 121.54) (width 1) (layer F.Cu) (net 49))
 (segment (start 111.8 116.1) (end 107.1 116.1) (width 1) (layer F.Cu) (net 49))
 (segment (start 114.6 113.3) (end 111.8 116.1) (width 1) (layer F.Cu) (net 49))
 (segment (start 115 110.18) (end 115 112.479998) (width 1) (layer F.Cu) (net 49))
 (segment (start 115 97.32) (end 115 96.1) (width 1) (layer F.Cu) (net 49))
 (segment (start 115 96.1) (end 115 105.1) (width 1) (layer F.Cu) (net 49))
 (segment (start 122.8 105.12) (end 115 97.32) (width 1) (layer F.Cu) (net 49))
 (segment (start 115 95.2) (end 115 96.1) (width 1) (layer F.Cu) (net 49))
 (segment (start 110.7 124.08) (end 110.7 126.7) (width 1) (layer F.Cu) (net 46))
 (segment (start 97.98 131.72) (end 98 131.7) (width 1) (layer F.Cu) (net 38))
 (segment (start 94.4 131.72) (end 97.98 131.72) (width 1) (layer F.Cu) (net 38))
 (segment (start 97.98 129.18) (end 98 129.16) (width 1) (layer F.Cu) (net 39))
 (segment (start 94.4 129.18) (end 97.98 129.18) (width 1) (layer F.Cu) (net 39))
 (segment (start 115.24 129.16) (end 115.28 129.12) (width 1) (layer F.Cu) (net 34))
 (segment (start 110.7 129.16) (end 115.24 129.16) (width 1) (layer F.Cu) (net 34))
 (segment (start 97.98 126.64) (end 98 126.62) (width 1) (layer F.Cu) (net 40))
 (segment (start 94.4 126.64) (end 97.98 126.64) (width 1) (layer F.Cu) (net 40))
 (segment (start 115.24 131.7) (end 115.28 131.66) (width 1) (layer F.Cu) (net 33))
 (segment (start 110.7 131.7) (end 115.24 131.7) (width 1) (layer F.Cu) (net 33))
 (segment (start 97.98 124.1) (end 98 124.08) (width 1) (layer F.Cu) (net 41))
 (segment (start 94.4 124.1) (end 97.98 124.1) (width 1) (layer F.Cu) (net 41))
 (segment (start 115.24 134.24) (end 115.28 134.2) (width 1) (layer F.Cu) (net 32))
 (segment (start 110.7 134.24) (end 115.24 134.24) (width 1) (layer F.Cu) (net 32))
 (segment (start 116.52 112.78) (end 110.7 112.78) (width 1) (layer B.Cu) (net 9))
 (segment (start 118.7 106.999998) (end 118.7 110.6) (width 1) (layer B.Cu) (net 9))
 (segment (start 124.9 100.4) (end 124.9 100.799998) (width 1) (layer B.Cu) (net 9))
 (segment (start 110.7 86.2) (end 124.9 100.4) (width 1) (layer B.Cu) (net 9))
 (segment (start 91.359998 86.2) (end 110.7 86.2) (width 1) (layer B.Cu) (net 9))
 (segment (start 78 99.559998) (end 91.359998 86.2) (width 1) (layer B.Cu) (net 9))
 (segment (start 118.7 110.6) (end 116.52 112.78) (width 1) (layer B.Cu) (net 9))
 (segment (start 124.9 100.799998) (end 118.7 106.999998) (width 1) (layer B.Cu) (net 9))
 (segment (start 78 100.3) (end 78 99.559998) (width 1) (layer B.Cu) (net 9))
 (segment (start 80.32 102.62) (end 78 100.3) (width 1) (layer B.Cu) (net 9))
 (segment (start 82.24 102.62) (end 80.32 102.62) (width 1) (layer B.Cu) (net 9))
 (segment (start 113.8 94.3) (end 113.8 96.6) (width 1) (layer B.Cu) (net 11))
 (segment (start 113.8 96.6) (end 112.86 97.54) (width 1) (layer B.Cu) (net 11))
 (segment (start 108.4 88.9) (end 113.8 94.3) (width 1) (layer B.Cu) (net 11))
 (segment (start 96.5 88.9) (end 108.4 88.9) (width 1) (layer B.Cu) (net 11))
 (segment (start 85.6 99.8) (end 96.5 88.9) (width 1) (layer B.Cu) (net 11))
 (segment (start 112.86 97.54) (end 110.7 97.54) (width 1) (layer B.Cu) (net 11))
 (segment (start 85.6 102.842928) (end 85.6 99.8) (width 1) (layer B.Cu) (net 11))
 (segment (start 83.44 105.002928) (end 85.6 102.842928) (width 1) (layer B.Cu) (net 11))
 (segment (start 83.44 105.16) (end 83.44 105.002928) (width 1) (layer B.Cu) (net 11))
 (segment (start 82.24 105.16) (end 83.44 105.16) (width 1) (layer B.Cu) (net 11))
 (segment (start 82.24 107.7) (end 85.5 107.7) (width 1) (layer B.Cu) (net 13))
 (segment (start 85.5 107.7) (end 88.1 105.1) (width 1) (layer B.Cu) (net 13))
 (segment (start 88.1 102.039998) (end 95.1 95.039998) (width 1) (layer B.Cu) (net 13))
 (segment (start 88.1 105.1) (end 88.1 102.039998) (width 1) (layer B.Cu) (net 13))
 (segment (start 95.1 95.039998) (end 95.1 93.7) (width 1) (layer B.Cu) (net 13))
 (segment (start 95.1 93.7) (end 98 90.8) (width 1) (layer B.Cu) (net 13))
 (segment (start 106.5 90.8) (end 110.7 95) (width 1) (layer B.Cu) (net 13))
 (segment (start 98 90.8) (end 106.5 90.8) (width 1) (layer B.Cu) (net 13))
 (segment (start 82.24 110.24) (end 85.24 110.24) (width 1) (layer B.Cu) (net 15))
 (segment (start 85.24 110.24) (end 87.6 112.6) (width 1) (layer B.Cu) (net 15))
 (segment (start 87.6 135.1) (end 91.09999 138.59999) (width 1) (layer B.Cu) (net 15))
 (segment (start 87.6 112.6) (end 87.6 135.1) (width 1) (layer B.Cu) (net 15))
 (segment (start 108.88001 138.59999) (end 110.7 136.78) (width 1) (layer B.Cu) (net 15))
 (segment (start 91.09999 138.59999) (end 108.88001 138.59999) (width 1) (layer B.Cu) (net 15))
 (segment (start 82.24 112.78) (end 77.5 117.52) (width 1) (layer B.Cu) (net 17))
 (segment (start 77.5 117.52) (end 77.5 134.2) (width 1) (layer B.Cu) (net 17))
 (segment (start 77.5 134.2) (end 91.5 148.2) (width 1) (layer B.Cu) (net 17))
 (segment (start 91.5 148.2) (end 110.6 148.2) (width 1) (layer B.Cu) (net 17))
 (segment (start 110.6 148.2) (end 119.4 139.4) (width 1) (layer B.Cu) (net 17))
 (segment (start 119.4 139.4) (end 119.4 123.1) (width 1) (layer B.Cu) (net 17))
 (segment (start 119.4 123.1) (end 113.3 117) (width 1) (layer B.Cu) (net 17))
 (segment (start 113.3 117) (end 108.9 117) (width 1) (layer B.Cu) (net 17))
 (segment (start 108.9 117) (end 107.6 118.3) (width 1) (layer B.Cu) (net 17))
 (segment (start 107.6 118.3) (end 107.6 120.2) (width 1) (layer B.Cu) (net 17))
 (segment (start 108.94 121.54) (end 110.7 121.54) (width 1) (layer B.Cu) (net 17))
 (segment (start 107.6 120.2) (end 108.94 121.54) (width 1) (layer B.Cu) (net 17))
 (segment (start 82.24 115.32) (end 79.5 118.06) (width 1) (layer B.Cu) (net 19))
 (segment (start 79.5 118.06) (end 79.5 134) (width 1) (layer B.Cu) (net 19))
 (segment (start 81.9 136.4) (end 85.2 136.4) (width 1) (layer B.Cu) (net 19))
 (segment (start 79.5 134) (end 81.9 136.4) (width 1) (layer B.Cu) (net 19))
 (segment (start 85.2 136.4) (end 89.4 140.6) (width 1) (layer B.Cu) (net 19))
 (segment (start 89.4 140.6) (end 113.1 140.6) (width 1) (layer B.Cu) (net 19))
 (segment (start 113.1 140.6) (end 117.1 136.6) (width 1) (layer B.Cu) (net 19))
 (segment (start 117.1 136.6) (end 117.1 136.5) (width 1) (layer B.Cu) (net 19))
 (segment (start 117.1 136.5) (end 117.5 136.1) (width 1) (layer B.Cu) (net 19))
 (segment (start 117.5 136.1) (end 117.5 124.1) (width 1) (layer B.Cu) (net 19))
 (segment (start 112.4 119) (end 110.7 119) (width 1) (layer B.Cu) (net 19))
 (segment (start 117.5 124.1) (end 112.4 119) (width 1) (layer B.Cu) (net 19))
 (segment (start 67 133.1) (end 66.98 133.08) (width 1) (layer F.Cu) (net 3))
 (segment (start 67 138.7) (end 71.5 143.2) (width 1) (layer F.Cu) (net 3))
 (segment (start 67 133.1) (end 67 138.7) (width 1) (layer F.Cu) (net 3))
 (segment (start 60.8 133.1) (end 67 133.1) (width 1) (layer F.Cu) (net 3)))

